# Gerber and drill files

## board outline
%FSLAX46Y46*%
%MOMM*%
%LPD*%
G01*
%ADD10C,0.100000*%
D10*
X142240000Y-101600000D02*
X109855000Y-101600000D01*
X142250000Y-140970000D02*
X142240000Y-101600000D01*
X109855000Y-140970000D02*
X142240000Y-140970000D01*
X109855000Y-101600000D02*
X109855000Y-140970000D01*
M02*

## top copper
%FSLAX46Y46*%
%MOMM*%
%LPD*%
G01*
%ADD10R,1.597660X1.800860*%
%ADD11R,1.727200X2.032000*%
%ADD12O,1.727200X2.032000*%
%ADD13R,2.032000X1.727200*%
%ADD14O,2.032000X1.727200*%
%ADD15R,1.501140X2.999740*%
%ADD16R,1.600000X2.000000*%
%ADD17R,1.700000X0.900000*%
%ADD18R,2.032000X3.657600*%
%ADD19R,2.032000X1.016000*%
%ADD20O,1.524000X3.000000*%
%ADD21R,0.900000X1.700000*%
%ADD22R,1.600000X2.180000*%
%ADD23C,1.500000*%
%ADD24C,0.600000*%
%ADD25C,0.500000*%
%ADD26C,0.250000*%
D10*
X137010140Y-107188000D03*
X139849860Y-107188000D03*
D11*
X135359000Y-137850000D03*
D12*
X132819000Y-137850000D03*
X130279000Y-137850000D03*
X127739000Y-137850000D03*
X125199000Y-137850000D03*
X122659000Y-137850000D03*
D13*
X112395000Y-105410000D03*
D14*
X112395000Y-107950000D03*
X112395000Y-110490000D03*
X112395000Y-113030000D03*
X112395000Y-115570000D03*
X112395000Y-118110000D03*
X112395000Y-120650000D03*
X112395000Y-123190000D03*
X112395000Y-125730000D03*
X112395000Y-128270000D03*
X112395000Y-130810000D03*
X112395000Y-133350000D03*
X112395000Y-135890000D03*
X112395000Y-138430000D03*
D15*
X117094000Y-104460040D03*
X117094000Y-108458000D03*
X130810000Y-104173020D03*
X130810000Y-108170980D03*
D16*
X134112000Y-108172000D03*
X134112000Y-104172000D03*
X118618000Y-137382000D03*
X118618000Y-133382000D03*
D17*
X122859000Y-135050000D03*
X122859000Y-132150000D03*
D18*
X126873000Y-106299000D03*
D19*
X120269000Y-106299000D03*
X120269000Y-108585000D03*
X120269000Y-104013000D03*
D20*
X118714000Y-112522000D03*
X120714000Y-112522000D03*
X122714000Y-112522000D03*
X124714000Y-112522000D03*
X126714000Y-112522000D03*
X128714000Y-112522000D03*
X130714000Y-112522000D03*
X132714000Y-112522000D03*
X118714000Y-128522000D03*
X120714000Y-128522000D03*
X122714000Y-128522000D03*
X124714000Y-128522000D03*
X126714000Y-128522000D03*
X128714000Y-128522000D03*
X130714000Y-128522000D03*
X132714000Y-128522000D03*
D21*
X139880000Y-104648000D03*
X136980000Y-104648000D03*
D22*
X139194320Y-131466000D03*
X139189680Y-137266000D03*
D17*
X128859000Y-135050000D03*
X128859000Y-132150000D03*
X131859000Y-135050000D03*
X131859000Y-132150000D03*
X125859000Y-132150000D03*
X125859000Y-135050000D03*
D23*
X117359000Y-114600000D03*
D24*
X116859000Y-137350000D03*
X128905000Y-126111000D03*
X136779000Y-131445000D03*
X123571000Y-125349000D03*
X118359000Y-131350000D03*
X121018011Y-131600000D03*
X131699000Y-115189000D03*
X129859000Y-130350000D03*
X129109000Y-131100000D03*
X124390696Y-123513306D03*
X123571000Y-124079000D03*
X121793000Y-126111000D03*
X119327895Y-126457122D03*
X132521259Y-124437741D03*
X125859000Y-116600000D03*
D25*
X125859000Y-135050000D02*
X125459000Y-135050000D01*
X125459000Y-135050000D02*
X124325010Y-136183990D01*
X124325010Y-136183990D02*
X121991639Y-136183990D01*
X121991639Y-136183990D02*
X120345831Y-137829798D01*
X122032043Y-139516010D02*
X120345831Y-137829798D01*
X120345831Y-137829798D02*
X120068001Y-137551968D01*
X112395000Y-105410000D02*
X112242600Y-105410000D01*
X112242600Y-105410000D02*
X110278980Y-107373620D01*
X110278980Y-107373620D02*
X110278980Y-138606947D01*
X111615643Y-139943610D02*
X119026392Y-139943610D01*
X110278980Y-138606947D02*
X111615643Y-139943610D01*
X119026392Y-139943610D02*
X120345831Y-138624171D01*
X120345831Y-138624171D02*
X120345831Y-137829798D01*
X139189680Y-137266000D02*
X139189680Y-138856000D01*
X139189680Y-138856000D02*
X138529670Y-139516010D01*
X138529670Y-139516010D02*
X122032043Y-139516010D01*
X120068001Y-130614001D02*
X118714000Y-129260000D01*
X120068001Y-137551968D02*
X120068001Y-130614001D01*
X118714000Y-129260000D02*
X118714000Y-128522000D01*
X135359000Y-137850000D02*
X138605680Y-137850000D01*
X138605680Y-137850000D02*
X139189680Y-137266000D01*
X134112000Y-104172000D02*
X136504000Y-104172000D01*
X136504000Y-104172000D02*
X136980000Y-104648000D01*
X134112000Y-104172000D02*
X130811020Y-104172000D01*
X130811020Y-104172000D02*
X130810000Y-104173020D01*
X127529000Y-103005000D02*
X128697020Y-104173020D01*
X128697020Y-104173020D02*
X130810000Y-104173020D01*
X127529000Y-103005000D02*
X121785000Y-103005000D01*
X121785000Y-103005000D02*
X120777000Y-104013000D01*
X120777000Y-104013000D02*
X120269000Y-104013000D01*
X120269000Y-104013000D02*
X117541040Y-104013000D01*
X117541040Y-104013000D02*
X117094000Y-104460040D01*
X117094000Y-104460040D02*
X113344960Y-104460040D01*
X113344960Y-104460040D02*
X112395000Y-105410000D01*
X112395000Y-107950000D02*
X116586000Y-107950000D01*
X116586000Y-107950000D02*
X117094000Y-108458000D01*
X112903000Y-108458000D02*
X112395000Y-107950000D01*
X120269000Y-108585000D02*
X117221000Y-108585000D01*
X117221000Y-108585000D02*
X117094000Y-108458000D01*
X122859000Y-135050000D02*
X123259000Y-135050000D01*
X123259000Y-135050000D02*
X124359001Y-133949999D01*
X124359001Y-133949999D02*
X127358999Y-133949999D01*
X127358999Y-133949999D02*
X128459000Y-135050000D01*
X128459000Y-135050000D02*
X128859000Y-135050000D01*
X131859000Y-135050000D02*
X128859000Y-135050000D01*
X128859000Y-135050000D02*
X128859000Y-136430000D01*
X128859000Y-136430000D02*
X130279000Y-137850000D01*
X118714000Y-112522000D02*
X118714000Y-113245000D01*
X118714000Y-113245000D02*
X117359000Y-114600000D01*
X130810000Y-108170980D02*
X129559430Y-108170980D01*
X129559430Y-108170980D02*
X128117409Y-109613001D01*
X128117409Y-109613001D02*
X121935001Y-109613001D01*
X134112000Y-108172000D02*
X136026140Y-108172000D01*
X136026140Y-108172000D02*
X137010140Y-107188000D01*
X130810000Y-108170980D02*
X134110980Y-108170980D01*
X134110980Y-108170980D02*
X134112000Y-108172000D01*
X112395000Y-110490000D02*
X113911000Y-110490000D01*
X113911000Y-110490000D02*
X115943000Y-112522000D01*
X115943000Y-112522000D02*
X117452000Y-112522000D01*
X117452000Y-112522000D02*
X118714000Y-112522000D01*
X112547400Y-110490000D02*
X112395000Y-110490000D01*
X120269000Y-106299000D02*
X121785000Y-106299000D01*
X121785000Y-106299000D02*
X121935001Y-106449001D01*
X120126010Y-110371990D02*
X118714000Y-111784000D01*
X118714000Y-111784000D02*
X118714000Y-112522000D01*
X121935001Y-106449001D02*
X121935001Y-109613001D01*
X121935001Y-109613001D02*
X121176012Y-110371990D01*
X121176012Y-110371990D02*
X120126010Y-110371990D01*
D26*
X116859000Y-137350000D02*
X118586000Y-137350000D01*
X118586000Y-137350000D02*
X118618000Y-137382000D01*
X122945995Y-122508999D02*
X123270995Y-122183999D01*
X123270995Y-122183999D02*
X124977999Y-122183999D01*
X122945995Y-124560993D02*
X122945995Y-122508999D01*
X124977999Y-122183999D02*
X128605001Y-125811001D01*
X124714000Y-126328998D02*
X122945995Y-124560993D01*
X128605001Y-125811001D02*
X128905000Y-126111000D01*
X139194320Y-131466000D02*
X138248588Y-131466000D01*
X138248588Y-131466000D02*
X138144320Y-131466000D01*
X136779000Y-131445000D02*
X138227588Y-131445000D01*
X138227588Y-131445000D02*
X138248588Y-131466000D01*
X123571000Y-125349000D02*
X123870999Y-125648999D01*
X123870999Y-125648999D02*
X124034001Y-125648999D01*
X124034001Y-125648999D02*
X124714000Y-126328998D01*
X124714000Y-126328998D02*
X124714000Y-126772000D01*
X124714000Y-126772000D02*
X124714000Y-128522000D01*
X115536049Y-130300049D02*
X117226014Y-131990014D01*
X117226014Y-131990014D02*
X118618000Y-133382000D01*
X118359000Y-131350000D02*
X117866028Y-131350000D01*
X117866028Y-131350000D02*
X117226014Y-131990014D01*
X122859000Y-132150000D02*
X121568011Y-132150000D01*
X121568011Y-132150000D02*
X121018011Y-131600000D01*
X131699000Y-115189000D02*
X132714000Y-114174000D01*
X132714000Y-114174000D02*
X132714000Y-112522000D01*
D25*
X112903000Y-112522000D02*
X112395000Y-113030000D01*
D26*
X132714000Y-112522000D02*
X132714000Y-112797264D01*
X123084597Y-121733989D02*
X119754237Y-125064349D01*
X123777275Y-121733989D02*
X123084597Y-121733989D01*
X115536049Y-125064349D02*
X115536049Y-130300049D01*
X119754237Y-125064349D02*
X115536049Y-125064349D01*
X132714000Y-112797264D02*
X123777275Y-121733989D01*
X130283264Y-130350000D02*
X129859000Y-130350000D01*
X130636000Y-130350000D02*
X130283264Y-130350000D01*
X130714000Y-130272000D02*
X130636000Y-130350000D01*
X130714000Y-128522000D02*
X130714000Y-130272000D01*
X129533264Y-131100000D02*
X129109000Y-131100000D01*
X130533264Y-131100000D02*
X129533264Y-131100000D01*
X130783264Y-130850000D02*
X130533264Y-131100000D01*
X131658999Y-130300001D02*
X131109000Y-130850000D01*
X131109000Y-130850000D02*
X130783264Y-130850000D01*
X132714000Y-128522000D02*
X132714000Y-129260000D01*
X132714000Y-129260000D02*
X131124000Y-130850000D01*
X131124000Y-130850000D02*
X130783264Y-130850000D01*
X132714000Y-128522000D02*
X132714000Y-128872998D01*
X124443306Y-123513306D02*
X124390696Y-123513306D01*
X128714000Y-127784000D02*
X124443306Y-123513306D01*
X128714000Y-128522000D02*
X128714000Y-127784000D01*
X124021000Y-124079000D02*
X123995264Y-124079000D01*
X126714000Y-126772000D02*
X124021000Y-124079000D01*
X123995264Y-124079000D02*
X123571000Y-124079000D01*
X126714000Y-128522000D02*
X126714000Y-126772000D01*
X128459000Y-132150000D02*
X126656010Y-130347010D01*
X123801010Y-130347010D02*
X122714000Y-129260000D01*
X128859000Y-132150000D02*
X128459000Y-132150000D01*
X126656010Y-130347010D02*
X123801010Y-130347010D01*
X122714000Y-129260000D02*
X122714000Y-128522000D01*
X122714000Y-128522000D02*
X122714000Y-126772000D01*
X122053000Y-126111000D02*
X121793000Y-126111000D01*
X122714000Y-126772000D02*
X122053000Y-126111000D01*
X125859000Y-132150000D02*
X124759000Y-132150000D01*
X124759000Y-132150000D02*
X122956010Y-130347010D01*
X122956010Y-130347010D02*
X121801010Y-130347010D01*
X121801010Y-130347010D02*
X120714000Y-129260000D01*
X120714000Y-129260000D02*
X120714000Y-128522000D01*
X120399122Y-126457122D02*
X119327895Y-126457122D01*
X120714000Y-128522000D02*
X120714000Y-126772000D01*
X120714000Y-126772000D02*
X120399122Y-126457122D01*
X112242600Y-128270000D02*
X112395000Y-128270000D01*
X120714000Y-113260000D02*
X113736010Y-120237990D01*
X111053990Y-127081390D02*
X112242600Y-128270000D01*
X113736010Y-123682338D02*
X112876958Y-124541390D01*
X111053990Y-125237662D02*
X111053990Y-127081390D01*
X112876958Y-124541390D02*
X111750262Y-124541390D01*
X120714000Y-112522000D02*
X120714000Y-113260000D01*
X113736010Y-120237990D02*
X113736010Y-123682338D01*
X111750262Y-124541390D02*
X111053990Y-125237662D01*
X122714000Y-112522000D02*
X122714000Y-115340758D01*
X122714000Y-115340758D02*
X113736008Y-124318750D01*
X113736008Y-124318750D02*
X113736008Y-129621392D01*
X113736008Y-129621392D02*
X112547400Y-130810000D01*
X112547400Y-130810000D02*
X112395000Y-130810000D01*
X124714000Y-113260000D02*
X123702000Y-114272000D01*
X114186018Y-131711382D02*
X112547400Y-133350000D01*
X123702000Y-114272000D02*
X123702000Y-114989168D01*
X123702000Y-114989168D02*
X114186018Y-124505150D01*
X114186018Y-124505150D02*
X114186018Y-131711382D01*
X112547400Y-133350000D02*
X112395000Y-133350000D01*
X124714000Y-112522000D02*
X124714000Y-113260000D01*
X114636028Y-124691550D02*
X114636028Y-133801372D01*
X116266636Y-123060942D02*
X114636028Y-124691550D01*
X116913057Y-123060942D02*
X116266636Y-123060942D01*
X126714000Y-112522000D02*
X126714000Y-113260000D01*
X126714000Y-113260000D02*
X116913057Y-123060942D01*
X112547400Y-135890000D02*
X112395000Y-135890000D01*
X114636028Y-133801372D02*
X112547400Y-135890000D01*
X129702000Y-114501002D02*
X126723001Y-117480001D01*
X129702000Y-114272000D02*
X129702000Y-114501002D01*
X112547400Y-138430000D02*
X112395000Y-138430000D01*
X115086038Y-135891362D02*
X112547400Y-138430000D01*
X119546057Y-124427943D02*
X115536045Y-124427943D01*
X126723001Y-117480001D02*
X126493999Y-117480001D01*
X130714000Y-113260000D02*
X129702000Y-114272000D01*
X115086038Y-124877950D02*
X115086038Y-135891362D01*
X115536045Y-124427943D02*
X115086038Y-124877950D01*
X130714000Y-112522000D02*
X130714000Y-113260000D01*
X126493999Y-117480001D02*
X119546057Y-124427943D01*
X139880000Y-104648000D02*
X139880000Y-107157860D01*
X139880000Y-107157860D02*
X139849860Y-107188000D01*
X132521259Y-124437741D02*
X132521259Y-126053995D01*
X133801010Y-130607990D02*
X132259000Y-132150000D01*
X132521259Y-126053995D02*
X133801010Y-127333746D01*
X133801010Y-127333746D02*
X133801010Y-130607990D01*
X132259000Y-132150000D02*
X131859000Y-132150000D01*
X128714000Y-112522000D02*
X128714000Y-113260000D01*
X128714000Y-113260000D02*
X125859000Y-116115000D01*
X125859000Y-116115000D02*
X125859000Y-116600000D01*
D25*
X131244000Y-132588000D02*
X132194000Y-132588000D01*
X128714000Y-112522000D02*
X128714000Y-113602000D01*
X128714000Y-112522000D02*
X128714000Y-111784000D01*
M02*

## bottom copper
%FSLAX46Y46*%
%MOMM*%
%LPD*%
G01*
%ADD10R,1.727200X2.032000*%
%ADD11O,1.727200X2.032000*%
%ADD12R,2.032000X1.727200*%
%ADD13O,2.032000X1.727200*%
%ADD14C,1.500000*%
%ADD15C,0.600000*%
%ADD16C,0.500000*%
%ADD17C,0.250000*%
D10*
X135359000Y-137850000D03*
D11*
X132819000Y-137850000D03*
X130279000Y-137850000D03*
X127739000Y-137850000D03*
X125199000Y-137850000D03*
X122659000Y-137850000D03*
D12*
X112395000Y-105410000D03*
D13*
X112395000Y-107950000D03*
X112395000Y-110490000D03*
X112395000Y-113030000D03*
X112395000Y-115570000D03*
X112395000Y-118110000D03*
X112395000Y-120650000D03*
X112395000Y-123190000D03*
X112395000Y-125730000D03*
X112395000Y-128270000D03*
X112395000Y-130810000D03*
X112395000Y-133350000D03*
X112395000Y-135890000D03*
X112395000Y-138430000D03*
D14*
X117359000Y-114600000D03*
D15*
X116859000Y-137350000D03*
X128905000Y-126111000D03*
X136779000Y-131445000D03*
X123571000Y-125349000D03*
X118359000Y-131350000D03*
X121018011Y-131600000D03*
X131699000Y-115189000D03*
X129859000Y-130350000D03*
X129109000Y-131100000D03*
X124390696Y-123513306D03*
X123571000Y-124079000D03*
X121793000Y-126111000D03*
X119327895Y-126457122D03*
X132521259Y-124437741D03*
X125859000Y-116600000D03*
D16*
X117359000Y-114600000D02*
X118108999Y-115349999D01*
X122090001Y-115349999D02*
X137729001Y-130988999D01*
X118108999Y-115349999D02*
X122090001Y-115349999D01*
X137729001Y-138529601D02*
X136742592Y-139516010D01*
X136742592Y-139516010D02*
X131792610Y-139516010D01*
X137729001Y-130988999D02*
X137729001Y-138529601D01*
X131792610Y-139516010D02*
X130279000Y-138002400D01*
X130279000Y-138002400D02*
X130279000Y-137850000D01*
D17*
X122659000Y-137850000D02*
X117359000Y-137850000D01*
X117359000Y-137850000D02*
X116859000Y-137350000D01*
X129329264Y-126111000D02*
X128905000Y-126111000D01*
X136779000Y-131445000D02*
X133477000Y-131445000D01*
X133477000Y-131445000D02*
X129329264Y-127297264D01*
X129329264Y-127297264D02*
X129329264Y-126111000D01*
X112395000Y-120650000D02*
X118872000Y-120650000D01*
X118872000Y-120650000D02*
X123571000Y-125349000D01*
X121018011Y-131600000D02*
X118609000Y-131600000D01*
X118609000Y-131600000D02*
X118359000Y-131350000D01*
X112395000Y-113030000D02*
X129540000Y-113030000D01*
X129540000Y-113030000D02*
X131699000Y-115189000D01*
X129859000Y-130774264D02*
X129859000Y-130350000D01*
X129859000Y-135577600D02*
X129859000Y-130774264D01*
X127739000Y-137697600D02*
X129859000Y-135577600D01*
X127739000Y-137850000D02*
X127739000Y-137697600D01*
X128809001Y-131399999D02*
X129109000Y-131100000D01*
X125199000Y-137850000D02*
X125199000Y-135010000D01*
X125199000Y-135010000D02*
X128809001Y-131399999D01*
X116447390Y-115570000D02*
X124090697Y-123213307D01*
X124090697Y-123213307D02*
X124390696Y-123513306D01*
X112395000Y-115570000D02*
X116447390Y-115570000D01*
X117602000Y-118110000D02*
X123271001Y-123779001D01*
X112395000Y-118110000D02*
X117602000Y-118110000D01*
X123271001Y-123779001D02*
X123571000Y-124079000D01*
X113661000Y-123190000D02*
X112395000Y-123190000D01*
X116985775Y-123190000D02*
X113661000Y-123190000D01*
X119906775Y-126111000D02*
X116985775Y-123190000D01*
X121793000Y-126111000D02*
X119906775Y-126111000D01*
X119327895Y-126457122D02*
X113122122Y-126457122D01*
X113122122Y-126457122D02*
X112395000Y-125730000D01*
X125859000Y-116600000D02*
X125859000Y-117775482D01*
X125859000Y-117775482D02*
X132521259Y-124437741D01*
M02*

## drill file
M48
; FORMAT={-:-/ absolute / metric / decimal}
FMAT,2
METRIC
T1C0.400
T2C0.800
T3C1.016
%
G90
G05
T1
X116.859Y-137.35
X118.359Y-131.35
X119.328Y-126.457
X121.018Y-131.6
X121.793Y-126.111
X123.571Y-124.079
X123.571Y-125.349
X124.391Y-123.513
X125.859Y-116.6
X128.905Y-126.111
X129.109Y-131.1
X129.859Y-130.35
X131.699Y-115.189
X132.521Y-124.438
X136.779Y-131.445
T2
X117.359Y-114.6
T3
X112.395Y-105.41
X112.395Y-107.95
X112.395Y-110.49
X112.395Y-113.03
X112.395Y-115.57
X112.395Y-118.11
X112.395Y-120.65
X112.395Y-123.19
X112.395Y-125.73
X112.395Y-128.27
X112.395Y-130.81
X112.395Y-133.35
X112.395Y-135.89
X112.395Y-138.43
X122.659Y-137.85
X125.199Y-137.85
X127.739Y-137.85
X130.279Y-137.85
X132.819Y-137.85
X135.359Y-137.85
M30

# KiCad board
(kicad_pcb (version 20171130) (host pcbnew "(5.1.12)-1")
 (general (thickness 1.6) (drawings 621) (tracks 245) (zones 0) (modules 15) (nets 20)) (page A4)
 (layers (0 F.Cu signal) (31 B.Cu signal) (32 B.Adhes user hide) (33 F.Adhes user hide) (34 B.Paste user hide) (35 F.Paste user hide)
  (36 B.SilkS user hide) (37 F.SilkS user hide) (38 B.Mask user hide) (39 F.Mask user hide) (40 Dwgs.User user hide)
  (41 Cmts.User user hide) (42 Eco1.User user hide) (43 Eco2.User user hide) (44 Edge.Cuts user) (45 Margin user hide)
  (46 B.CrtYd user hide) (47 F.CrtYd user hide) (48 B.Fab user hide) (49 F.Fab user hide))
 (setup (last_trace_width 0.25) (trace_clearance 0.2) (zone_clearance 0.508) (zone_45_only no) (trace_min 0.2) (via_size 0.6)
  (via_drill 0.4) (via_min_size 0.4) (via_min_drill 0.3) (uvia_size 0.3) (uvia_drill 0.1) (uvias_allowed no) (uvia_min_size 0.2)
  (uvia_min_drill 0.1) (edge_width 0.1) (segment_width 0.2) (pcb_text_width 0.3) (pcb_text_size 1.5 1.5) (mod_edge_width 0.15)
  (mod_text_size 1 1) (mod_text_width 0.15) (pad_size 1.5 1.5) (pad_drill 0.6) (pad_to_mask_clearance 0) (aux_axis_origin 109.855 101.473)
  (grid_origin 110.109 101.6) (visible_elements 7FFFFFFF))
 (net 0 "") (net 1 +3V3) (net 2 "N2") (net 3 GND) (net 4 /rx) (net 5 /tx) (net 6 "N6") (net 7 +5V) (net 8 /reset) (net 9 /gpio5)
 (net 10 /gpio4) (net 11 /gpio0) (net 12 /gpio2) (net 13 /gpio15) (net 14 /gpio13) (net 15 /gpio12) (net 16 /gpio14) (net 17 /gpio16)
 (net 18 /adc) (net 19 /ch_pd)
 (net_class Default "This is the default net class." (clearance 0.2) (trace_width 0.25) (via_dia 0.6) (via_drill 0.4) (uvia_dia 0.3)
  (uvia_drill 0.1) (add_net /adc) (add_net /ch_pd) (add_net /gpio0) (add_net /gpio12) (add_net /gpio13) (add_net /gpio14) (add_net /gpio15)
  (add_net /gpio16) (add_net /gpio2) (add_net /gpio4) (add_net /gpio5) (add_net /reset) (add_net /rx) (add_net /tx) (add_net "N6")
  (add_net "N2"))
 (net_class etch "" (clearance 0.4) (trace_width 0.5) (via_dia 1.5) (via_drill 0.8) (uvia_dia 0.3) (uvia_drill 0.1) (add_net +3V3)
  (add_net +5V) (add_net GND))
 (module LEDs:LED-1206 (layer F.Cu) (at 138.43 107.188 180)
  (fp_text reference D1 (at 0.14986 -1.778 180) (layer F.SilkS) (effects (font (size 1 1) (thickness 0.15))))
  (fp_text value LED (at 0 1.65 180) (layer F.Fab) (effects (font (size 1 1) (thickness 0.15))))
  (pad 2 smd rect (at 1.41986 0) (size 1.59766 1.80086) (layers F.Cu F.Paste F.Mask) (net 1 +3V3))
  (pad 1 smd rect (at -1.41986 0) (size 1.59766 1.80086) (layers F.Cu F.Paste F.Mask) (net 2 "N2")))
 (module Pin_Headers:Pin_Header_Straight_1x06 (layer F.Cu) (at 135.359 137.85 270)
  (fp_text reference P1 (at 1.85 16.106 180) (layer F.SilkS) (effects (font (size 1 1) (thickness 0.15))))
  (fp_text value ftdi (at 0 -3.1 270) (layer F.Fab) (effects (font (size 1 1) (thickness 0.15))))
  (pad 1 thru_hole rect (at 0 0 270) (size 2.032 1.7272) (drill 1.016) (layers *.Cu *.Mask F.SilkS) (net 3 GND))
  (pad 2 thru_hole oval (at 0 2.54 270) (size 2.032 1.7272) (drill 1.016) (layers *.Cu *.Mask F.SilkS))
  (pad 3 thru_hole oval (at 0 5.08 270) (size 2.032 1.7272) (drill 1.016) (layers *.Cu *.Mask F.SilkS) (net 1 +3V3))
  (pad 4 thru_hole oval (at 0 7.62 270) (size 2.032 1.7272) (drill 1.016) (layers *.Cu *.Mask F.SilkS) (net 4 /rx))
  (pad 5 thru_hole oval (at 0 10.16 270) (size 2.032 1.7272) (drill 1.016) (layers *.Cu *.Mask F.SilkS) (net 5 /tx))
  (pad 6 thru_hole oval (at 0 12.7 270) (size 2.032 1.7272) (drill 1.016) (layers *.Cu *.Mask F.SilkS) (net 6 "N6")))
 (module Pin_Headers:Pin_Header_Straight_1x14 (layer B.Cu) (at 112.395 105.41 180)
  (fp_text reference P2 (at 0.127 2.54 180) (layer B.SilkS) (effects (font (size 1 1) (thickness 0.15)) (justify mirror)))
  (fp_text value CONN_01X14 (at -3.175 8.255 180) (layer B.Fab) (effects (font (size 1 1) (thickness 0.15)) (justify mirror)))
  (pad 1 thru_hole rect (at 0 0 180) (size 2.032 1.7272) (drill 1.016) (layers *.Cu *.Mask B.SilkS) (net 3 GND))
  (pad 2 thru_hole oval (at 0 -2.54 180) (size 2.032 1.7272) (drill 1.016) (layers *.Cu *.Mask B.SilkS) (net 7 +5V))
  (pad 3 thru_hole oval (at 0 -5.08 180) (size 2.032 1.7272) (drill 1.016) (layers *.Cu *.Mask B.SilkS) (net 1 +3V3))
  (pad 4 thru_hole oval (at 0 -7.62 180) (size 2.032 1.7272) (drill 1.016) (layers *.Cu *.Mask B.SilkS) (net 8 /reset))
  (pad 5 thru_hole oval (at 0 -10.16 180) (size 2.032 1.7272) (drill 1.016) (layers *.Cu *.Mask B.SilkS) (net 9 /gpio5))
  (pad 6 thru_hole oval (at 0 -12.7 180) (size 2.032 1.7272) (drill 1.016) (layers *.Cu *.Mask B.SilkS) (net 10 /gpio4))
  (pad 7 thru_hole oval (at 0 -15.24 180) (size 2.032 1.7272) (drill 1.016) (layers *.Cu *.Mask B.SilkS) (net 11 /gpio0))
  (pad 8 thru_hole oval (at 0 -17.78 180) (size 2.032 1.7272) (drill 1.016) (layers *.Cu *.Mask B.SilkS) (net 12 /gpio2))
  (pad 9 thru_hole oval (at 0 -20.32 180) (size 2.032 1.7272) (drill 1.016) (layers *.Cu *.Mask B.SilkS) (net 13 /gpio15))
  (pad 10 thru_hole oval (at 0 -22.86 180) (size 2.032 1.7272) (drill 1.016) (layers *.Cu *.Mask B.SilkS) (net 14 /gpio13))
  (pad 11 thru_hole oval (at 0 -25.4 180) (size 2.032 1.7272) (drill 1.016) (layers *.Cu *.Mask B.SilkS) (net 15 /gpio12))
  (pad 12 thru_hole oval (at 0 -27.94 180) (size 2.032 1.7272) (drill 1.016) (layers *.Cu *.Mask B.SilkS) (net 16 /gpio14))
  (pad 13 thru_hole oval (at 0 -30.48 180) (size 2.032 1.7272) (drill 1.016) (layers *.Cu *.Mask B.SilkS) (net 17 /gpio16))
  (pad 14 thru_hole oval (at 0 -33.02 180) (size 2.032 1.7272) (drill 1.016) (layers *.Cu *.Mask B.SilkS) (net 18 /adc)))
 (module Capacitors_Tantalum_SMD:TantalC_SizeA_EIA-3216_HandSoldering (layer F.Cu) (at 117.094 106.45902 90)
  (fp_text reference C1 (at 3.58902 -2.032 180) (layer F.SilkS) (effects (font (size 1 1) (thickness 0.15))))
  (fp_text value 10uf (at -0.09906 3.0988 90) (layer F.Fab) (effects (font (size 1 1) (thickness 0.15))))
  (pad 2 smd rect (at 1.99898 0 90) (size 2.99974 1.50114) (layers F.Cu F.Paste F.Mask) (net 3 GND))
  (pad 1 smd rect (at -1.99898 0 90) (size 2.99974 1.50114) (layers F.Cu F.Paste F.Mask) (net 7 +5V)))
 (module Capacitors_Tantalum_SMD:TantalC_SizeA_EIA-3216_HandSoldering (layer F.Cu) (at 130.81 106.172 90)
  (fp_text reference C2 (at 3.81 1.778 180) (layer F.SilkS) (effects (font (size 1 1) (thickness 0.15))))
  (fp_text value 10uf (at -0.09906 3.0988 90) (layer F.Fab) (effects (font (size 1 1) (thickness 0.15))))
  (pad 2 smd rect (at 1.99898 0 90) (size 2.99974 1.50114) (layers F.Cu F.Paste F.Mask) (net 3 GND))
  (pad 1 smd rect (at -1.99898 0 90) (size 2.99974 1.50114) (layers F.Cu F.Paste F.Mask) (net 1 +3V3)))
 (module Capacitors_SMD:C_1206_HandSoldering (layer F.Cu) (at 134.112 106.172 90)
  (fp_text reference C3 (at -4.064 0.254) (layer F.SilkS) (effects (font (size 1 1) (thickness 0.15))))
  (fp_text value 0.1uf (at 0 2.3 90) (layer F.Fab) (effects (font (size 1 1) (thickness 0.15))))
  (pad 1 smd rect (at -2 0 90) (size 2 1.6) (layers F.Cu F.Paste F.Mask) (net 1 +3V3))
  (pad 2 smd rect (at 2 0 90) (size 2 1.6) (layers F.Cu F.Paste F.Mask) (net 3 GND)))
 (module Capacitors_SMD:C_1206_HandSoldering (layer F.Cu) (at 118.618 135.382 90)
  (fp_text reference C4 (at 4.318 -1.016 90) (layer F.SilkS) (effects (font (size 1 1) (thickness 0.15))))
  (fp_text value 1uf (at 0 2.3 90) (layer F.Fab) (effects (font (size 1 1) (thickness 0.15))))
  (pad 1 smd rect (at -2 0 90) (size 2 1.6) (layers F.Cu F.Paste F.Mask) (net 6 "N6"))
  (pad 2 smd rect (at 2 0 90) (size 2 1.6) (layers F.Cu F.Paste F.Mask) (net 8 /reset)))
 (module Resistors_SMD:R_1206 (layer F.Cu) (at 122.859 133.6 90)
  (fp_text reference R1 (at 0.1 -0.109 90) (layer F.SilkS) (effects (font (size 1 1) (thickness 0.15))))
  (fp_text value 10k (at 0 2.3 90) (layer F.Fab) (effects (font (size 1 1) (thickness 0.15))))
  (pad 1 smd rect (at -1.45 0 90) (size 0.9 1.7) (layers F.Cu F.Paste F.Mask) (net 1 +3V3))
  (pad 2 smd rect (at 1.45 0 90) (size 0.9 1.7) (layers F.Cu F.Paste F.Mask) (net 8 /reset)))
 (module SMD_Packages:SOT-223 (layer F.Cu) (at 123.571 106.299 270)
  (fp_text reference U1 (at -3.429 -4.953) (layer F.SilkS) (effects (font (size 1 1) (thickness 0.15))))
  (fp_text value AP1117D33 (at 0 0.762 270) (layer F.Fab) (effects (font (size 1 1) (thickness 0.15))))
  (pad 4 smd rect (at 0 -3.302 270) (size 3.6576 2.032) (layers F.Cu F.Paste F.Mask))
  (pad 2 smd rect (at 0 3.302 270) (size 1.016 2.032) (layers F.Cu F.Paste F.Mask) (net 1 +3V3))
  (pad 3 smd rect (at 2.286 3.302 270) (size 1.016 2.032) (layers F.Cu F.Paste F.Mask) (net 7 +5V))
  (pad 1 smd rect (at -2.286 3.302 270) (size 1.016 2.032) (layers F.Cu F.Paste F.Mask) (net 3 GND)))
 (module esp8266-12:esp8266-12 (layer F.Cu) (at 118.714 112.622)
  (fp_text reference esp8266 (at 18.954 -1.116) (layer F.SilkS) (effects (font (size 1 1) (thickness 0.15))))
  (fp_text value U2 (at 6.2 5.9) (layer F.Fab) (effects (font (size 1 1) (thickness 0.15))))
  (pad 8 smd oval (at 0 -0.1) (size 1.524 3) (layers F.Cu F.Paste F.Mask) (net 1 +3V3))
  (pad 7 smd oval (at 2 -0.1) (size 1.524 3) (layers F.Cu F.Paste F.Mask) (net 14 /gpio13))
  (pad 6 smd oval (at 4 -0.1) (size 1.524 3) (layers F.Cu F.Paste F.Mask) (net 15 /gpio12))
  (pad 5 smd oval (at 6 -0.1) (size 1.524 3) (layers F.Cu F.Paste F.Mask) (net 16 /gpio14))
  (pad 4 smd oval (at 8 -0.1) (size 1.524 3) (layers F.Cu F.Paste F.Mask) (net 17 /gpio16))
  (pad 3 smd oval (at 10 -0.1) (size 1.524 3) (layers F.Cu F.Paste F.Mask) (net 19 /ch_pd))
  (pad 2 smd oval (at 12 -0.1) (size 1.524 3) (layers F.Cu F.Paste F.Mask) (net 18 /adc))
  (pad 1 smd oval (at 14 -0.1) (size 1.524 3) (layers F.Cu F.Paste F.Mask) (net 8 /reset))
  (pad 9 smd oval (at 0 15.9) (size 1.524 3) (layers F.Cu F.Paste F.Mask) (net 3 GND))
  (pad 10 smd oval (at 2 15.9) (size 1.524 3) (layers F.Cu F.Paste F.Mask) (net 13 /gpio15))
  (pad 11 smd oval (at 4 15.9) (size 1.524 3) (layers F.Cu F.Paste F.Mask) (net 12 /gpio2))
  (pad 12 smd oval (at 6 15.9) (size 1.524 3) (layers F.Cu F.Paste F.Mask) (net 11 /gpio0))
  (pad 13 smd oval (at 8 15.9) (size 1.524 3) (layers F.Cu F.Paste F.Mask) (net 10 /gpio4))
  (pad 14 smd oval (at 10 15.9) (size 1.524 3) (layers F.Cu F.Paste F.Mask) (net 9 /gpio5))
  (pad 15 smd oval (at 12 15.9) (size 1.524 3) (layers F.Cu F.Paste F.Mask) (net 4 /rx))
  (pad 16 smd oval (at 14 15.9) (size 1.524 3) (layers F.Cu F.Paste F.Mask) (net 5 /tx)))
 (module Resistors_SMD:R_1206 (layer F.Cu) (at 138.43 104.648 180)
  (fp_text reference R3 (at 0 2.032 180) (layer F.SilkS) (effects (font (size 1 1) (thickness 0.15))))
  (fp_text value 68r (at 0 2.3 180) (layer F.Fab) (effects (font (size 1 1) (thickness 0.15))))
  (pad 1 smd rect (at -1.45 0 180) (size 0.9 1.7) (layers F.Cu F.Paste F.Mask) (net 2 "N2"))
  (pad 2 smd rect (at 1.45 0 180) (size 0.9 1.7) (layers F.Cu F.Paste F.Mask) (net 3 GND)))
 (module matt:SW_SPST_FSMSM (layer F.Cu) (at 139.192 134.366 270)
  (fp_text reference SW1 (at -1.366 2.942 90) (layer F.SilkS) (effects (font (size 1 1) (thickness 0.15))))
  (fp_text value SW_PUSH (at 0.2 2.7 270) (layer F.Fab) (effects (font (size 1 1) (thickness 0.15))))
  (pad 1 smd rect (at -2.9 -0.00232 270) (size 2.18 1.6) (layers F.Cu F.Paste F.Mask) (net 11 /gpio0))
  (pad 2 smd rect (at 2.9 0.00232 270) (size 2.18 1.6) (layers F.Cu F.Paste F.Mask) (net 3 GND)))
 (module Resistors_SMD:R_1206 (layer F.Cu) (at 128.859 133.6 90)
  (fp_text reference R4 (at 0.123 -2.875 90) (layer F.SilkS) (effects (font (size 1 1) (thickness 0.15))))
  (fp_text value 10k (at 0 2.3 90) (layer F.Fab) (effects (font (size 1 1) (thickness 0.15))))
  (pad 1 smd rect (at -1.45 0 90) (size 0.9 1.7) (layers F.Cu F.Paste F.Mask) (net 1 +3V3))
  (pad 2 smd rect (at 1.45 0 90) (size 0.9 1.7) (layers F.Cu F.Paste F.Mask) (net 12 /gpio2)))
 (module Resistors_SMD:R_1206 (layer F.Cu) (at 131.859 133.6 90)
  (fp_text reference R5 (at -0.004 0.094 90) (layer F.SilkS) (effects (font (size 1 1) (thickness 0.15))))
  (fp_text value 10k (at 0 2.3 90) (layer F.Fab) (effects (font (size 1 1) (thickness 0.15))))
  (pad 1 smd rect (at -1.45 0 90) (size 0.9 1.7) (layers F.Cu F.Paste F.Mask) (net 1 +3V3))
  (pad 2 smd rect (at 1.45 0 90) (size 0.9 1.7) (layers F.Cu F.Paste F.Mask) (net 19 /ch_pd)))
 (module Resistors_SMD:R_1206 (layer F.Cu) (at 125.859 133.6 270)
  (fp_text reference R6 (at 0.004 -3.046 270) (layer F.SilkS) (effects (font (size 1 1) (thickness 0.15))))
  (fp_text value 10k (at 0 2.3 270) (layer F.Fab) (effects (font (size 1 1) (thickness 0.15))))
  (pad 1 smd rect (at -1.45 0 270) (size 0.9 1.7) (layers F.Cu F.Paste F.Mask) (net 13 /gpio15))
  (pad 2 smd rect (at 1.45 0 270) (size 0.9 1.7) (layers F.Cu F.Paste F.Mask) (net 3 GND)))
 (gr_line (start 142.24 101.6) (end 109.855 101.6) (layer Edge.Cuts) (width 0.1))
 (gr_line (start 142.25 140.97) (end 142.24 101.6) (layer Edge.Cuts) (width 0.1))
 (gr_line (start 109.855 140.97) (end 142.24 140.97) (layer Edge.Cuts) (width 0.1))
 (gr_line (start 109.855 101.6) (end 109.855 140.97) (layer Edge.Cuts) (width 0.1))
 (segment (start 125.859 135.05) (end 125.459 135.05) (width 0.5) (layer F.Cu) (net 3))
 (segment (start 125.459 135.05) (end 124.32501 136.18399) (width 0.5) (layer F.Cu) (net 3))
 (segment (start 124.32501 136.18399) (end 121.991639 136.18399) (width 0.5) (layer F.Cu) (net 3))
 (segment (start 121.991639 136.18399) (end 120.345831 137.829798) (width 0.5) (layer F.Cu) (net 3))
 (segment (start 122.032043 139.51601) (end 120.345831 137.829798) (width 0.5) (layer F.Cu) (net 3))
 (segment (start 120.345831 137.829798) (end 120.068001 137.551968) (width 0.5) (layer F.Cu) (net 3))
 (segment (start 112.395 105.41) (end 112.2426 105.41) (width 0.5) (layer F.Cu) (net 3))
 (segment (start 112.2426 105.41) (end 110.27898 107.37362) (width 0.5) (layer F.Cu) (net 3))
 (segment (start 110.27898 107.37362) (end 110.27898 138.606947) (width 0.5) (layer F.Cu) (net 3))
 (segment (start 111.615643 139.94361) (end 119.026392 139.94361) (width 0.5) (layer F.Cu) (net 3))
 (segment (start 110.27898 138.606947) (end 111.615643 139.94361) (width 0.5) (layer F.Cu) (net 3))
 (segment (start 119.026392 139.94361) (end 120.345831 138.624171) (width 0.5) (layer F.Cu) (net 3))
 (segment (start 120.345831 138.624171) (end 120.345831 137.829798) (width 0.5) (layer F.Cu) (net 3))
 (segment (start 139.18968 137.266) (end 139.18968 138.856) (width 0.5) (layer F.Cu) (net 3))
 (segment (start 139.18968 138.856) (end 138.52967 139.51601) (width 0.5) (layer F.Cu) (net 3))
 (segment (start 138.52967 139.51601) (end 122.032043 139.51601) (width 0.5) (layer F.Cu) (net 3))
 (segment (start 120.068001 130.614001) (end 118.714 129.26) (width 0.5) (layer F.Cu) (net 3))
 (segment (start 120.068001 137.551968) (end 120.068001 130.614001) (width 0.5) (layer F.Cu) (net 3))
 (segment (start 118.714 129.26) (end 118.714 128.522) (width 0.5) (layer F.Cu) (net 3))
 (segment (start 135.359 137.85) (end 138.60568 137.85) (width 0.5) (layer F.Cu) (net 3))
 (segment (start 138.60568 137.85) (end 139.18968 137.266) (width 0.5) (layer F.Cu) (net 3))
 (segment (start 134.112 104.172) (end 136.504 104.172) (width 0.5) (layer F.Cu) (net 3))
 (segment (start 136.504 104.172) (end 136.98 104.648) (width 0.5) (layer F.Cu) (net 3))
 (segment (start 134.112 104.172) (end 130.81102 104.172) (width 0.5) (layer F.Cu) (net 3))
 (segment (start 130.81102 104.172) (end 130.81 104.17302) (width 0.5) (layer F.Cu) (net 3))
 (segment (start 127.529 103.005) (end 128.69702 104.17302) (width 0.5) (layer F.Cu) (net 3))
 (segment (start 128.69702 104.17302) (end 130.81 104.17302) (width 0.5) (layer F.Cu) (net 3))
 (segment (start 127.529 103.005) (end 121.785 103.005) (width 0.5) (layer F.Cu) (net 3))
 (segment (start 121.785 103.005) (end 120.777 104.013) (width 0.5) (layer F.Cu) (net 3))
 (segment (start 120.777 104.013) (end 120.269 104.013) (width 0.5) (layer F.Cu) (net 3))
 (segment (start 120.269 104.013) (end 117.54104 104.013) (width 0.5) (layer F.Cu) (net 3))
 (segment (start 117.54104 104.013) (end 117.094 104.46004) (width 0.5) (layer F.Cu) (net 3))
 (segment (start 117.094 104.46004) (end 113.34496 104.46004) (width 0.5) (layer F.Cu) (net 3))
 (segment (start 113.34496 104.46004) (end 112.395 105.41) (width 0.5) (layer F.Cu) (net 3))
 (segment (start 112.395 107.95) (end 116.586 107.95) (width 0.5) (layer F.Cu) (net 7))
 (segment (start 116.586 107.95) (end 117.094 108.458) (width 0.5) (layer F.Cu) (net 7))
 (segment (start 112.903 108.458) (end 112.395 107.95) (width 0.5) (layer F.Cu) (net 7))
 (segment (start 120.269 108.585) (end 117.221 108.585) (width 0.5) (layer F.Cu) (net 7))
 (segment (start 117.221 108.585) (end 117.094 108.458) (width 0.5) (layer F.Cu) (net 7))
 (segment (start 122.859 135.05) (end 123.259 135.05) (width 0.5) (layer F.Cu) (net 1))
 (segment (start 123.259 135.05) (end 124.359001 133.949999) (width 0.5) (layer F.Cu) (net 1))
 (segment (start 124.359001 133.949999) (end 127.358999 133.949999) (width 0.5) (layer F.Cu) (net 1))
 (segment (start 127.358999 133.949999) (end 128.459 135.05) (width 0.5) (layer F.Cu) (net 1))
 (segment (start 128.459 135.05) (end 128.859 135.05) (width 0.5) (layer F.Cu) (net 1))
 (segment (start 131.859 135.05) (end 128.859 135.05) (width 0.5) (layer F.Cu) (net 1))
 (segment (start 128.859 135.05) (end 128.859 136.43) (width 0.5) (layer F.Cu) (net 1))
 (segment (start 128.859 136.43) (end 130.279 137.85) (width 0.5) (layer F.Cu) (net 1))
 (segment (start 117.359 114.6) (end 118.108999 115.349999) (width 0.5) (layer B.Cu) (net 1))
 (segment (start 122.090001 115.349999) (end 137.729001 130.988999) (width 0.5) (layer B.Cu) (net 1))
 (segment (start 118.108999 115.349999) (end 122.090001 115.349999) (width 0.5) (layer B.Cu) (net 1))
 (segment (start 137.729001 138.529601) (end 136.742592 139.51601) (width 0.5) (layer B.Cu) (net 1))
 (segment (start 136.742592 139.51601) (end 131.79261 139.51601) (width 0.5) (layer B.Cu) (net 1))
 (segment (start 137.729001 130.988999) (end 137.729001 138.529601) (width 0.5) (layer B.Cu) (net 1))
 (segment (start 131.79261 139.51601) (end 130.279 138.0024) (width 0.5) (layer B.Cu) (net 1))
 (segment (start 130.279 138.0024) (end 130.279 137.85) (width 0.5) (layer B.Cu) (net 1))
 (segment (start 118.714 112.522) (end 118.714 113.245) (width 0.5) (layer F.Cu) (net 1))
 (segment (start 118.714 113.245) (end 117.359 114.6) (width 0.5) (layer F.Cu) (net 1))
 (segment (start 130.81 108.17098) (end 129.55943 108.17098) (width 0.5) (layer F.Cu) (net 1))
 (segment (start 129.55943 108.17098) (end 128.117409 109.613001) (width 0.5) (layer F.Cu) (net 1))
 (segment (start 128.117409 109.613001) (end 121.935001 109.613001) (width 0.5) (layer F.Cu) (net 1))
 (segment (start 134.112 108.172) (end 136.02614 108.172) (width 0.5) (layer F.Cu) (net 1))
 (segment (start 136.02614 108.172) (end 137.01014 107.188) (width 0.5) (layer F.Cu) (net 1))
 (segment (start 130.81 108.17098) (end 134.11098 108.17098) (width 0.5) (layer F.Cu) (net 1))
 (segment (start 134.11098 108.17098) (end 134.112 108.172) (width 0.5) (layer F.Cu) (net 1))
 (segment (start 112.395 110.49) (end 113.911 110.49) (width 0.5) (layer F.Cu) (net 1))
 (segment (start 113.911 110.49) (end 115.943 112.522) (width 0.5) (layer F.Cu) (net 1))
 (segment (start 115.943 112.522) (end 117.452 112.522) (width 0.5) (layer F.Cu) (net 1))
 (segment (start 117.452 112.522) (end 118.714 112.522) (width 0.5) (layer F.Cu) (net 1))
 (segment (start 112.5474 110.49) (end 112.395 110.49) (width 0.5) (layer F.Cu) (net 1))
 (segment (start 120.269 106.299) (end 121.785 106.299) (width 0.5) (layer F.Cu) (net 1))
 (segment (start 121.785 106.299) (end 121.935001 106.449001) (width 0.5) (layer F.Cu) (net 1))
 (segment (start 120.12601 110.37199) (end 118.714 111.784) (width 0.5) (layer F.Cu) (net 1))
 (segment (start 118.714 111.784) (end 118.714 112.522) (width 0.5) (layer F.Cu) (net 1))
 (segment (start 121.935001 106.449001) (end 121.935001 109.613001) (width 0.5) (layer F.Cu) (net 1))
 (segment (start 121.935001 109.613001) (end 121.176012 110.37199) (width 0.5) (layer F.Cu) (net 1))
 (segment (start 121.176012 110.37199) (end 120.12601 110.37199) (width 0.5) (layer F.Cu) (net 1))
 (segment (start 116.859 137.35) (end 118.586 137.35) (width 0.25) (layer F.Cu) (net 6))
 (segment (start 118.586 137.35) (end 118.618 137.382) (width 0.25) (layer F.Cu) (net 6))
 (segment (start 122.659 137.85) (end 117.359 137.85) (width 0.25) (layer B.Cu) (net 6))
 (segment (start 117.359 137.85) (end 116.859 137.35) (width 0.25) (layer B.Cu) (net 6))
 (segment (start 122.945995 122.508999) (end 123.270995 122.183999) (width 0.25) (layer F.Cu) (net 11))
 (segment (start 123.270995 122.183999) (end 124.977999 122.183999) (width 0.25) (layer F.Cu) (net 11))
 (segment (start 122.945995 124.560993) (end 122.945995 122.508999) (width 0.25) (layer F.Cu) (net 11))
 (segment (start 124.977999 122.183999) (end 128.605001 125.811001) (width 0.25) (layer F.Cu) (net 11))
 (segment (start 124.714 126.328998) (end 122.945995 124.560993) (width 0.25) (layer F.Cu) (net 11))
 (segment (start 128.605001 125.811001) (end 128.905 126.111) (width 0.25) (layer F.Cu) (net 11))
 (segment (start 129.329264 126.111) (end 128.905 126.111) (width 0.25) (layer B.Cu) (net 11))
 (segment (start 136.779 131.445) (end 133.477 131.445) (width 0.25) (layer B.Cu) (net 11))
 (segment (start 133.477 131.445) (end 129.329264 127.297264) (width 0.25) (layer B.Cu) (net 11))
 (segment (start 129.329264 127.297264) (end 129.329264 126.111) (width 0.25) (layer B.Cu) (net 11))
 (segment (start 139.19432 131.466) (end 138.248588 131.466) (width 0.25) (layer F.Cu) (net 11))
 (segment (start 138.248588 131.466) (end 138.14432 131.466) (width 0.25) (layer F.Cu) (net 11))
 (segment (start 136.779 131.445) (end 138.227588 131.445) (width 0.25) (layer F.Cu) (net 11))
 (segment (start 138.227588 131.445) (end 138.248588 131.466) (width 0.25) (layer F.Cu) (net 11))
 (segment (start 123.571 125.349) (end 123.870999 125.648999) (width 0.25) (layer F.Cu) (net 11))
 (segment (start 123.870999 125.648999) (end 124.034001 125.648999) (width 0.25) (layer F.Cu) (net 11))
 (segment (start 124.034001 125.648999) (end 124.714 126.328998) (width 0.25) (layer F.Cu) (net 11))
 (segment (start 112.395 120.65) (end 118.872 120.65) (width 0.25) (layer B.Cu) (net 11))
 (segment (start 118.872 120.65) (end 123.571 125.349) (width 0.25) (layer B.Cu) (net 11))
 (segment (start 124.714 126.328998) (end 124.714 126.772) (width 0.25) (layer F.Cu) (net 11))
 (segment (start 124.714 126.772) (end 124.714 128.522) (width 0.25) (layer F.Cu) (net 11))
 (segment (start 115.536049 130.300049) (end 117.226014 131.990014) (width 0.25) (layer F.Cu) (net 8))
 (segment (start 117.226014 131.990014) (end 118.618 133.382) (width 0.25) (layer F.Cu) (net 8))
 (segment (start 118.359 131.35) (end 117.866028 131.35) (width 0.25) (layer F.Cu) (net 8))
 (segment (start 117.866028 131.35) (end 117.226014 131.990014) (width 0.25) (layer F.Cu) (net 8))
 (segment (start 121.018011 131.6) (end 118.609 131.6) (width 0.25) (layer B.Cu) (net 8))
 (segment (start 118.609 131.6) (end 118.359 131.35) (width 0.25) (layer B.Cu) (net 8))
 (segment (start 122.859 132.15) (end 121.568011 132.15) (width 0.25) (layer F.Cu) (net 8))
 (segment (start 121.568011 132.15) (end 121.018011 131.6) (width 0.25) (layer F.Cu) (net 8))
 (segment (start 131.699 115.189) (end 132.714 114.174) (width 0.25) (layer F.Cu) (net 8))
 (segment (start 132.714 114.174) (end 132.714 112.522) (width 0.25) (layer F.Cu) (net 8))
 (segment (start 112.395 113.03) (end 129.54 113.03) (width 0.25) (layer B.Cu) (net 8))
 (segment (start 129.54 113.03) (end 131.699 115.189) (width 0.25) (layer B.Cu) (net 8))
 (segment (start 112.903 112.522) (end 112.395 113.03) (width 0.5) (layer F.Cu) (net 8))
 (segment (start 132.714 112.522) (end 132.714 112.797264) (width 0.25) (layer F.Cu) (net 8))
 (segment (start 123.084597 121.733989) (end 119.754237 125.064349) (width 0.25) (layer F.Cu) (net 8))
 (segment (start 123.777275 121.733989) (end 123.084597 121.733989) (width 0.25) (layer F.Cu) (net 8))
 (segment (start 115.536049 125.064349) (end 115.536049 130.300049) (width 0.25) (layer F.Cu) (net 8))
 (segment (start 119.754237 125.064349) (end 115.536049 125.064349) (width 0.25) (layer F.Cu) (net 8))
 (segment (start 132.714 112.797264) (end 123.777275 121.733989) (width 0.25) (layer F.Cu) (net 8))
 (segment (start 129.859 130.774264) (end 129.859 130.35) (width 0.25) (layer B.Cu) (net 4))
 (segment (start 129.859 135.5776) (end 129.859 130.774264) (width 0.25) (layer B.Cu) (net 4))
 (segment (start 127.739 137.6976) (end 129.859 135.5776) (width 0.25) (layer B.Cu) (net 4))
 (segment (start 130.283264 130.35) (end 129.859 130.35) (width 0.25) (layer F.Cu) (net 4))
 (segment (start 130.636 130.35) (end 130.283264 130.35) (width 0.25) (layer F.Cu) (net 4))
 (segment (start 127.739 137.85) (end 127.739 137.6976) (width 0.25) (layer B.Cu) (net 4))
 (segment (start 130.714 130.272) (end 130.636 130.35) (width 0.25) (layer F.Cu) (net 4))
 (segment (start 130.714 128.522) (end 130.714 130.272) (width 0.25) (layer F.Cu) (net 4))
 (segment (start 128.809001 131.399999) (end 129.109 131.1) (width 0.25) (layer B.Cu) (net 5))
 (segment (start 125.199 137.85) (end 125.199 135.01) (width 0.25) (layer B.Cu) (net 5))
 (segment (start 125.199 135.01) (end 128.809001 131.399999) (width 0.25) (layer B.Cu) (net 5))
 (segment (start 129.533264 131.1) (end 129.109 131.1) (width 0.25) (layer F.Cu) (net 5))
 (segment (start 130.533264 131.1) (end 129.533264 131.1) (width 0.25) (layer F.Cu) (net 5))
 (segment (start 130.783264 130.85) (end 130.533264 131.1) (width 0.25) (layer F.Cu) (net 5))
 (segment (start 131.658999 130.300001) (end 131.109 130.85) (width 0.25) (layer F.Cu) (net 5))
 (segment (start 131.109 130.85) (end 130.783264 130.85) (width 0.25) (layer F.Cu) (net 5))
 (segment (start 132.714 128.522) (end 132.714 129.26) (width 0.25) (layer F.Cu) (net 5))
 (segment (start 132.714 129.26) (end 131.124 130.85) (width 0.25) (layer F.Cu) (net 5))
 (segment (start 131.124 130.85) (end 130.783264 130.85) (width 0.25) (layer F.Cu) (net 5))
 (segment (start 132.714 128.522) (end 132.714 128.872998) (width 0.25) (layer F.Cu) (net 5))
 (segment (start 124.443306 123.513306) (end 124.390696 123.513306) (width 0.25) (layer F.Cu) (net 9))
 (segment (start 128.714 127.784) (end 124.443306 123.513306) (width 0.25) (layer F.Cu) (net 9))
 (segment (start 116.44739 115.57) (end 124.090697 123.213307) (width 0.25) (layer B.Cu) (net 9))
 (segment (start 128.714 128.522) (end 128.714 127.784) (width 0.25) (layer F.Cu) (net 9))
 (segment (start 124.090697 123.213307) (end 124.390696 123.513306) (width 0.25) (layer B.Cu) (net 9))
 (segment (start 112.395 115.57) (end 116.44739 115.57) (width 0.25) (layer B.Cu) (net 9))
 (segment (start 117.602 118.11) (end 123.271001 123.779001) (width 0.25) (layer B.Cu) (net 10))
 (segment (start 112.395 118.11) (end 117.602 118.11) (width 0.25) (layer B.Cu) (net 10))
 (segment (start 124.021 124.079) (end 123.995264 124.079) (width 0.25) (layer F.Cu) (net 10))
 (segment (start 126.714 126.772) (end 124.021 124.079) (width 0.25) (layer F.Cu) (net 10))
 (segment (start 123.995264 124.079) (end 123.571 124.079) (width 0.25) (layer F.Cu) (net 10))
 (segment (start 123.271001 123.779001) (end 123.571 124.079) (width 0.25) (layer B.Cu) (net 10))
 (segment (start 126.714 128.522) (end 126.714 126.772) (width 0.25) (layer F.Cu) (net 10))
 (segment (start 128.459 132.15) (end 126.65601 130.34701) (width 0.25) (layer F.Cu) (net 12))
 (segment (start 123.80101 130.34701) (end 122.714 129.26) (width 0.25) (layer F.Cu) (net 12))
 (segment (start 128.859 132.15) (end 128.459 132.15) (width 0.25) (layer F.Cu) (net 12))
 (segment (start 126.65601 130.34701) (end 123.80101 130.34701) (width 0.25) (layer F.Cu) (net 12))
 (segment (start 122.714 129.26) (end 122.714 128.522) (width 0.25) (layer F.Cu) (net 12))
 (segment (start 113.661 123.19) (end 112.395 123.19) (width 0.25) (layer B.Cu) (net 12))
 (segment (start 116.985775 123.19) (end 113.661 123.19) (width 0.25) (layer B.Cu) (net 12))
 (segment (start 119.906775 126.111) (end 116.985775 123.19) (width 0.25) (layer B.Cu) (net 12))
 (segment (start 121.793 126.111) (end 119.906775 126.111) (width 0.25) (layer B.Cu) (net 12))
 (segment (start 122.714 128.522) (end 122.714 126.772) (width 0.25) (layer F.Cu) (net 12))
 (segment (start 122.053 126.111) (end 121.793 126.111) (width 0.25) (layer F.Cu) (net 12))
 (segment (start 122.714 126.772) (end 122.053 126.111) (width 0.25) (layer F.Cu) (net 12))
 (segment (start 125.859 132.15) (end 124.759 132.15) (width 0.25) (layer F.Cu) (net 13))
 (segment (start 124.759 132.15) (end 122.95601 130.34701) (width 0.25) (layer F.Cu) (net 13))
 (segment (start 122.95601 130.34701) (end 121.80101 130.34701) (width 0.25) (layer F.Cu) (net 13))
 (segment (start 121.80101 130.34701) (end 120.714 129.26) (width 0.25) (layer F.Cu) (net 13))
 (segment (start 120.714 129.26) (end 120.714 128.522) (width 0.25) (layer F.Cu) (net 13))
 (segment (start 119.327895 126.457122) (end 113.122122 126.457122) (width 0.25) (layer B.Cu) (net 13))
 (segment (start 113.122122 126.457122) (end 112.395 125.73) (width 0.25) (layer B.Cu) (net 13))
 (segment (start 120.399122 126.457122) (end 119.327895 126.457122) (width 0.25) (layer F.Cu) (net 13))
 (segment (start 120.714 128.522) (end 120.714 126.772) (width 0.25) (layer F.Cu) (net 13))
 (segment (start 120.714 126.772) (end 120.399122 126.457122) (width 0.25) (layer F.Cu) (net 13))
 (segment (start 112.2426 128.27) (end 112.395 128.27) (width 0.25) (layer F.Cu) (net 14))
 (segment (start 120.714 113.26) (end 113.73601 120.23799) (width 0.25) (layer F.Cu) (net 14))
 (segment (start 111.05399 127.08139) (end 112.2426 128.27) (width 0.25) (layer F.Cu) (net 14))
 (segment (start 113.73601 123.682338) (end 112.876958 124.54139) (width 0.25) (layer F.Cu) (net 14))
 (segment (start 111.05399 125.237662) (end 111.05399 127.08139) (width 0.25) (layer F.Cu) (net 14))
 (segment (start 112.876958 124.54139) (end 111.750262 124.54139) (width 0.25) (layer F.Cu) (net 14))
 (segment (start 120.714 112.522) (end 120.714 113.26) (width 0.25) (layer F.Cu) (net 14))
 (segment (start 113.73601 120.23799) (end 113.73601 123.682338) (width 0.25) (layer F.Cu) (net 14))
 (segment (start 111.750262 124.54139) (end 111.05399 125.237662) (width 0.25) (layer F.Cu) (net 14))
 (segment (start 122.714 112.522) (end 122.714 115.340758) (width 0.25) (layer F.Cu) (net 15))
 (segment (start 122.714 115.340758) (end 113.736008 124.31875) (width 0.25) (layer F.Cu) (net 15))
 (segment (start 113.736008 124.31875) (end 113.736008 129.621392) (width 0.25) (layer F.Cu) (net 15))
 (segment (start 113.736008 129.621392) (end 112.5474 130.81) (width 0.25) (layer F.Cu) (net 15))
 (segment (start 112.5474 130.81) (end 112.395 130.81) (width 0.25) (layer F.Cu) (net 15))
 (segment (start 124.714 113.26) (end 123.702 114.272) (width 0.25) (layer F.Cu) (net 16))
 (segment (start 114.186018 131.711382) (end 112.5474 133.35) (width 0.25) (layer F.Cu) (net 16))
 (segment (start 123.702 114.272) (end 123.702 114.989168) (width 0.25) (layer F.Cu) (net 16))
 (segment (start 123.702 114.989168) (end 114.186018 124.50515) (width 0.25) (layer F.Cu) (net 16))
 (segment (start 114.186018 124.50515) (end 114.186018 131.711382) (width 0.25) (layer F.Cu) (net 16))
 (segment (start 112.5474 133.35) (end 112.395 133.35) (width 0.25) (layer F.Cu) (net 16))
 (segment (start 124.714 112.522) (end 124.714 113.26) (width 0.25) (layer F.Cu) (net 16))
 (segment (start 114.636028 124.69155) (end 114.636028 133.801372) (width 0.25) (layer F.Cu) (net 17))
 (segment (start 116.266636 123.060942) (end 114.636028 124.69155) (width 0.25) (layer F.Cu) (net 17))
 (segment (start 116.913057 123.060942) (end 116.266636 123.060942) (width 0.25) (layer F.Cu) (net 17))
 (segment (start 126.714 112.522) (end 126.714 113.26) (width 0.25) (layer F.Cu) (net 17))
 (segment (start 126.714 113.26) (end 116.913057 123.060942) (width 0.25) (layer F.Cu) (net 17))
 (segment (start 112.5474 135.89) (end 112.395 135.89) (width 0.25) (layer F.Cu) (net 17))
 (segment (start 114.636028 133.801372) (end 112.5474 135.89) (width 0.25) (layer F.Cu) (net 17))
 (segment (start 129.702 114.501002) (end 126.723001 117.480001) (width 0.25) (layer F.Cu) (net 18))
 (segment (start 129.702 114.272) (end 129.702 114.501002) (width 0.25) (layer F.Cu) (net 18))
 (segment (start 112.5474 138.43) (end 112.395 138.43) (width 0.25) (layer F.Cu) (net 18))
 (segment (start 115.086038 135.891362) (end 112.5474 138.43) (width 0.25) (layer F.Cu) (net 18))
 (segment (start 119.546057 124.427943) (end 115.536045 124.427943) (width 0.25) (layer F.Cu) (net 18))
 (segment (start 126.723001 117.480001) (end 126.493999 117.480001) (width 0.25) (layer F.Cu) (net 18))
 (segment (start 130.714 113.26) (end 129.702 114.272) (width 0.25) (layer F.Cu) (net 18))
 (segment (start 115.086038 124.87795) (end 115.086038 135.891362) (width 0.25) (layer F.Cu) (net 18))
 (segment (start 115.536045 124.427943) (end 115.086038 124.87795) (width 0.25) (layer F.Cu) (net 18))
 (segment (start 130.714 112.522) (end 130.714 113.26) (width 0.25) (layer F.Cu) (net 18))
 (segment (start 126.493999 117.480001) (end 119.546057 124.427943) (width 0.25) (layer F.Cu) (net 18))
 (segment (start 139.88 104.648) (end 139.88 107.15786) (width 0.25) (layer F.Cu) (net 2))
 (segment (start 139.88 107.15786) (end 139.84986 107.188) (width 0.25) (layer F.Cu) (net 2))
 (segment (start 132.521259 124.437741) (end 132.521259 126.053995) (width 0.25) (layer F.Cu) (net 19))
 (segment (start 133.80101 130.60799) (end 132.259 132.15) (width 0.25) (layer F.Cu) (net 19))
 (segment (start 132.521259 126.053995) (end 133.80101 127.333746) (width 0.25) (layer F.Cu) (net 19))
 (segment (start 133.80101 127.333746) (end 133.80101 130.60799) (width 0.25) (layer F.Cu) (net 19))
 (segment (start 132.259 132.15) (end 131.859 132.15) (width 0.25) (layer F.Cu) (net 19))
 (segment (start 125.859 116.6) (end 125.859 117.775482) (width 0.25) (layer B.Cu) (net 19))
 (segment (start 125.859 117.775482) (end 132.521259 124.437741) (width 0.25) (layer B.Cu) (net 19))
 (segment (start 128.714 112.522) (end 128.714 113.26) (width 0.25) (layer F.Cu) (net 19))
 (segment (start 128.714 113.26) (end 125.859 116.115) (width 0.25) (layer F.Cu) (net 19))
 (segment (start 125.859 116.115) (end 125.859 116.6) (width 0.25) (layer F.Cu) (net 19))
 (segment (start 131.244 132.588) (end 132.194 132.588) (width 0.5) (layer F.Cu) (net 19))
 (segment (start 128.714 112.522) (end 128.714 113.602) (width 0.5) (layer F.Cu) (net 19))
 (segment (start 128.714 112.522) (end 128.714 111.784) (width 0.5) (layer F.Cu) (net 19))
 (via (at 117.359 114.6) (size 1.5) (drill 0.8) (layers F.Cu B.Cu) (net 1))
 (via (at 116.859 137.35) (size 0.6) (drill 0.4) (layers F.Cu B.Cu) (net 6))
 (via (at 128.905 126.111) (size 0.6) (drill 0.4) (layers F.Cu B.Cu) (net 11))
 (via (at 136.779 131.445) (size 0.6) (drill 0.4) (layers F.Cu B.Cu) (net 11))
 (via (at 123.571 125.349) (size 0.6) (drill 0.4) (layers F.Cu B.Cu) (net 11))
 (via (at 118.359 131.35) (size 0.6) (drill 0.4) (layers F.Cu B.Cu) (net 8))
 (via (at 121.018011 131.6) (size 0.6) (drill 0.4) (layers F.Cu B.Cu) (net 8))
 (via (at 131.699 115.189) (size 0.6) (drill 0.4) (layers F.Cu B.Cu) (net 8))
 (via (at 129.859 130.35) (size 0.6) (drill 0.4) (layers F.Cu B.Cu) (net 4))
 (via (at 129.109 131.1) (size 0.6) (drill 0.4) (layers F.Cu B.Cu) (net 5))
 (via (at 124.390696 123.513306) (size 0.6) (drill 0.4) (layers F.Cu B.Cu) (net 9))
 (via (at 123.571 124.079) (size 0.6) (drill 0.4) (layers F.Cu B.Cu) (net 10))
 (via (at 121.793 126.111) (size 0.6) (drill 0.4) (layers F.Cu B.Cu) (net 12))
 (via (at 119.327895 126.457122) (size 0.6) (drill 0.4) (layers F.Cu B.Cu) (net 13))
 (via (at 132.521259 124.437741) (size 0.6) (drill 0.4) (layers F.Cu B.Cu) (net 19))
 (via (at 125.859 116.6) (size 0.6) (drill 0.4) (layers F.Cu B.Cu) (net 19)))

